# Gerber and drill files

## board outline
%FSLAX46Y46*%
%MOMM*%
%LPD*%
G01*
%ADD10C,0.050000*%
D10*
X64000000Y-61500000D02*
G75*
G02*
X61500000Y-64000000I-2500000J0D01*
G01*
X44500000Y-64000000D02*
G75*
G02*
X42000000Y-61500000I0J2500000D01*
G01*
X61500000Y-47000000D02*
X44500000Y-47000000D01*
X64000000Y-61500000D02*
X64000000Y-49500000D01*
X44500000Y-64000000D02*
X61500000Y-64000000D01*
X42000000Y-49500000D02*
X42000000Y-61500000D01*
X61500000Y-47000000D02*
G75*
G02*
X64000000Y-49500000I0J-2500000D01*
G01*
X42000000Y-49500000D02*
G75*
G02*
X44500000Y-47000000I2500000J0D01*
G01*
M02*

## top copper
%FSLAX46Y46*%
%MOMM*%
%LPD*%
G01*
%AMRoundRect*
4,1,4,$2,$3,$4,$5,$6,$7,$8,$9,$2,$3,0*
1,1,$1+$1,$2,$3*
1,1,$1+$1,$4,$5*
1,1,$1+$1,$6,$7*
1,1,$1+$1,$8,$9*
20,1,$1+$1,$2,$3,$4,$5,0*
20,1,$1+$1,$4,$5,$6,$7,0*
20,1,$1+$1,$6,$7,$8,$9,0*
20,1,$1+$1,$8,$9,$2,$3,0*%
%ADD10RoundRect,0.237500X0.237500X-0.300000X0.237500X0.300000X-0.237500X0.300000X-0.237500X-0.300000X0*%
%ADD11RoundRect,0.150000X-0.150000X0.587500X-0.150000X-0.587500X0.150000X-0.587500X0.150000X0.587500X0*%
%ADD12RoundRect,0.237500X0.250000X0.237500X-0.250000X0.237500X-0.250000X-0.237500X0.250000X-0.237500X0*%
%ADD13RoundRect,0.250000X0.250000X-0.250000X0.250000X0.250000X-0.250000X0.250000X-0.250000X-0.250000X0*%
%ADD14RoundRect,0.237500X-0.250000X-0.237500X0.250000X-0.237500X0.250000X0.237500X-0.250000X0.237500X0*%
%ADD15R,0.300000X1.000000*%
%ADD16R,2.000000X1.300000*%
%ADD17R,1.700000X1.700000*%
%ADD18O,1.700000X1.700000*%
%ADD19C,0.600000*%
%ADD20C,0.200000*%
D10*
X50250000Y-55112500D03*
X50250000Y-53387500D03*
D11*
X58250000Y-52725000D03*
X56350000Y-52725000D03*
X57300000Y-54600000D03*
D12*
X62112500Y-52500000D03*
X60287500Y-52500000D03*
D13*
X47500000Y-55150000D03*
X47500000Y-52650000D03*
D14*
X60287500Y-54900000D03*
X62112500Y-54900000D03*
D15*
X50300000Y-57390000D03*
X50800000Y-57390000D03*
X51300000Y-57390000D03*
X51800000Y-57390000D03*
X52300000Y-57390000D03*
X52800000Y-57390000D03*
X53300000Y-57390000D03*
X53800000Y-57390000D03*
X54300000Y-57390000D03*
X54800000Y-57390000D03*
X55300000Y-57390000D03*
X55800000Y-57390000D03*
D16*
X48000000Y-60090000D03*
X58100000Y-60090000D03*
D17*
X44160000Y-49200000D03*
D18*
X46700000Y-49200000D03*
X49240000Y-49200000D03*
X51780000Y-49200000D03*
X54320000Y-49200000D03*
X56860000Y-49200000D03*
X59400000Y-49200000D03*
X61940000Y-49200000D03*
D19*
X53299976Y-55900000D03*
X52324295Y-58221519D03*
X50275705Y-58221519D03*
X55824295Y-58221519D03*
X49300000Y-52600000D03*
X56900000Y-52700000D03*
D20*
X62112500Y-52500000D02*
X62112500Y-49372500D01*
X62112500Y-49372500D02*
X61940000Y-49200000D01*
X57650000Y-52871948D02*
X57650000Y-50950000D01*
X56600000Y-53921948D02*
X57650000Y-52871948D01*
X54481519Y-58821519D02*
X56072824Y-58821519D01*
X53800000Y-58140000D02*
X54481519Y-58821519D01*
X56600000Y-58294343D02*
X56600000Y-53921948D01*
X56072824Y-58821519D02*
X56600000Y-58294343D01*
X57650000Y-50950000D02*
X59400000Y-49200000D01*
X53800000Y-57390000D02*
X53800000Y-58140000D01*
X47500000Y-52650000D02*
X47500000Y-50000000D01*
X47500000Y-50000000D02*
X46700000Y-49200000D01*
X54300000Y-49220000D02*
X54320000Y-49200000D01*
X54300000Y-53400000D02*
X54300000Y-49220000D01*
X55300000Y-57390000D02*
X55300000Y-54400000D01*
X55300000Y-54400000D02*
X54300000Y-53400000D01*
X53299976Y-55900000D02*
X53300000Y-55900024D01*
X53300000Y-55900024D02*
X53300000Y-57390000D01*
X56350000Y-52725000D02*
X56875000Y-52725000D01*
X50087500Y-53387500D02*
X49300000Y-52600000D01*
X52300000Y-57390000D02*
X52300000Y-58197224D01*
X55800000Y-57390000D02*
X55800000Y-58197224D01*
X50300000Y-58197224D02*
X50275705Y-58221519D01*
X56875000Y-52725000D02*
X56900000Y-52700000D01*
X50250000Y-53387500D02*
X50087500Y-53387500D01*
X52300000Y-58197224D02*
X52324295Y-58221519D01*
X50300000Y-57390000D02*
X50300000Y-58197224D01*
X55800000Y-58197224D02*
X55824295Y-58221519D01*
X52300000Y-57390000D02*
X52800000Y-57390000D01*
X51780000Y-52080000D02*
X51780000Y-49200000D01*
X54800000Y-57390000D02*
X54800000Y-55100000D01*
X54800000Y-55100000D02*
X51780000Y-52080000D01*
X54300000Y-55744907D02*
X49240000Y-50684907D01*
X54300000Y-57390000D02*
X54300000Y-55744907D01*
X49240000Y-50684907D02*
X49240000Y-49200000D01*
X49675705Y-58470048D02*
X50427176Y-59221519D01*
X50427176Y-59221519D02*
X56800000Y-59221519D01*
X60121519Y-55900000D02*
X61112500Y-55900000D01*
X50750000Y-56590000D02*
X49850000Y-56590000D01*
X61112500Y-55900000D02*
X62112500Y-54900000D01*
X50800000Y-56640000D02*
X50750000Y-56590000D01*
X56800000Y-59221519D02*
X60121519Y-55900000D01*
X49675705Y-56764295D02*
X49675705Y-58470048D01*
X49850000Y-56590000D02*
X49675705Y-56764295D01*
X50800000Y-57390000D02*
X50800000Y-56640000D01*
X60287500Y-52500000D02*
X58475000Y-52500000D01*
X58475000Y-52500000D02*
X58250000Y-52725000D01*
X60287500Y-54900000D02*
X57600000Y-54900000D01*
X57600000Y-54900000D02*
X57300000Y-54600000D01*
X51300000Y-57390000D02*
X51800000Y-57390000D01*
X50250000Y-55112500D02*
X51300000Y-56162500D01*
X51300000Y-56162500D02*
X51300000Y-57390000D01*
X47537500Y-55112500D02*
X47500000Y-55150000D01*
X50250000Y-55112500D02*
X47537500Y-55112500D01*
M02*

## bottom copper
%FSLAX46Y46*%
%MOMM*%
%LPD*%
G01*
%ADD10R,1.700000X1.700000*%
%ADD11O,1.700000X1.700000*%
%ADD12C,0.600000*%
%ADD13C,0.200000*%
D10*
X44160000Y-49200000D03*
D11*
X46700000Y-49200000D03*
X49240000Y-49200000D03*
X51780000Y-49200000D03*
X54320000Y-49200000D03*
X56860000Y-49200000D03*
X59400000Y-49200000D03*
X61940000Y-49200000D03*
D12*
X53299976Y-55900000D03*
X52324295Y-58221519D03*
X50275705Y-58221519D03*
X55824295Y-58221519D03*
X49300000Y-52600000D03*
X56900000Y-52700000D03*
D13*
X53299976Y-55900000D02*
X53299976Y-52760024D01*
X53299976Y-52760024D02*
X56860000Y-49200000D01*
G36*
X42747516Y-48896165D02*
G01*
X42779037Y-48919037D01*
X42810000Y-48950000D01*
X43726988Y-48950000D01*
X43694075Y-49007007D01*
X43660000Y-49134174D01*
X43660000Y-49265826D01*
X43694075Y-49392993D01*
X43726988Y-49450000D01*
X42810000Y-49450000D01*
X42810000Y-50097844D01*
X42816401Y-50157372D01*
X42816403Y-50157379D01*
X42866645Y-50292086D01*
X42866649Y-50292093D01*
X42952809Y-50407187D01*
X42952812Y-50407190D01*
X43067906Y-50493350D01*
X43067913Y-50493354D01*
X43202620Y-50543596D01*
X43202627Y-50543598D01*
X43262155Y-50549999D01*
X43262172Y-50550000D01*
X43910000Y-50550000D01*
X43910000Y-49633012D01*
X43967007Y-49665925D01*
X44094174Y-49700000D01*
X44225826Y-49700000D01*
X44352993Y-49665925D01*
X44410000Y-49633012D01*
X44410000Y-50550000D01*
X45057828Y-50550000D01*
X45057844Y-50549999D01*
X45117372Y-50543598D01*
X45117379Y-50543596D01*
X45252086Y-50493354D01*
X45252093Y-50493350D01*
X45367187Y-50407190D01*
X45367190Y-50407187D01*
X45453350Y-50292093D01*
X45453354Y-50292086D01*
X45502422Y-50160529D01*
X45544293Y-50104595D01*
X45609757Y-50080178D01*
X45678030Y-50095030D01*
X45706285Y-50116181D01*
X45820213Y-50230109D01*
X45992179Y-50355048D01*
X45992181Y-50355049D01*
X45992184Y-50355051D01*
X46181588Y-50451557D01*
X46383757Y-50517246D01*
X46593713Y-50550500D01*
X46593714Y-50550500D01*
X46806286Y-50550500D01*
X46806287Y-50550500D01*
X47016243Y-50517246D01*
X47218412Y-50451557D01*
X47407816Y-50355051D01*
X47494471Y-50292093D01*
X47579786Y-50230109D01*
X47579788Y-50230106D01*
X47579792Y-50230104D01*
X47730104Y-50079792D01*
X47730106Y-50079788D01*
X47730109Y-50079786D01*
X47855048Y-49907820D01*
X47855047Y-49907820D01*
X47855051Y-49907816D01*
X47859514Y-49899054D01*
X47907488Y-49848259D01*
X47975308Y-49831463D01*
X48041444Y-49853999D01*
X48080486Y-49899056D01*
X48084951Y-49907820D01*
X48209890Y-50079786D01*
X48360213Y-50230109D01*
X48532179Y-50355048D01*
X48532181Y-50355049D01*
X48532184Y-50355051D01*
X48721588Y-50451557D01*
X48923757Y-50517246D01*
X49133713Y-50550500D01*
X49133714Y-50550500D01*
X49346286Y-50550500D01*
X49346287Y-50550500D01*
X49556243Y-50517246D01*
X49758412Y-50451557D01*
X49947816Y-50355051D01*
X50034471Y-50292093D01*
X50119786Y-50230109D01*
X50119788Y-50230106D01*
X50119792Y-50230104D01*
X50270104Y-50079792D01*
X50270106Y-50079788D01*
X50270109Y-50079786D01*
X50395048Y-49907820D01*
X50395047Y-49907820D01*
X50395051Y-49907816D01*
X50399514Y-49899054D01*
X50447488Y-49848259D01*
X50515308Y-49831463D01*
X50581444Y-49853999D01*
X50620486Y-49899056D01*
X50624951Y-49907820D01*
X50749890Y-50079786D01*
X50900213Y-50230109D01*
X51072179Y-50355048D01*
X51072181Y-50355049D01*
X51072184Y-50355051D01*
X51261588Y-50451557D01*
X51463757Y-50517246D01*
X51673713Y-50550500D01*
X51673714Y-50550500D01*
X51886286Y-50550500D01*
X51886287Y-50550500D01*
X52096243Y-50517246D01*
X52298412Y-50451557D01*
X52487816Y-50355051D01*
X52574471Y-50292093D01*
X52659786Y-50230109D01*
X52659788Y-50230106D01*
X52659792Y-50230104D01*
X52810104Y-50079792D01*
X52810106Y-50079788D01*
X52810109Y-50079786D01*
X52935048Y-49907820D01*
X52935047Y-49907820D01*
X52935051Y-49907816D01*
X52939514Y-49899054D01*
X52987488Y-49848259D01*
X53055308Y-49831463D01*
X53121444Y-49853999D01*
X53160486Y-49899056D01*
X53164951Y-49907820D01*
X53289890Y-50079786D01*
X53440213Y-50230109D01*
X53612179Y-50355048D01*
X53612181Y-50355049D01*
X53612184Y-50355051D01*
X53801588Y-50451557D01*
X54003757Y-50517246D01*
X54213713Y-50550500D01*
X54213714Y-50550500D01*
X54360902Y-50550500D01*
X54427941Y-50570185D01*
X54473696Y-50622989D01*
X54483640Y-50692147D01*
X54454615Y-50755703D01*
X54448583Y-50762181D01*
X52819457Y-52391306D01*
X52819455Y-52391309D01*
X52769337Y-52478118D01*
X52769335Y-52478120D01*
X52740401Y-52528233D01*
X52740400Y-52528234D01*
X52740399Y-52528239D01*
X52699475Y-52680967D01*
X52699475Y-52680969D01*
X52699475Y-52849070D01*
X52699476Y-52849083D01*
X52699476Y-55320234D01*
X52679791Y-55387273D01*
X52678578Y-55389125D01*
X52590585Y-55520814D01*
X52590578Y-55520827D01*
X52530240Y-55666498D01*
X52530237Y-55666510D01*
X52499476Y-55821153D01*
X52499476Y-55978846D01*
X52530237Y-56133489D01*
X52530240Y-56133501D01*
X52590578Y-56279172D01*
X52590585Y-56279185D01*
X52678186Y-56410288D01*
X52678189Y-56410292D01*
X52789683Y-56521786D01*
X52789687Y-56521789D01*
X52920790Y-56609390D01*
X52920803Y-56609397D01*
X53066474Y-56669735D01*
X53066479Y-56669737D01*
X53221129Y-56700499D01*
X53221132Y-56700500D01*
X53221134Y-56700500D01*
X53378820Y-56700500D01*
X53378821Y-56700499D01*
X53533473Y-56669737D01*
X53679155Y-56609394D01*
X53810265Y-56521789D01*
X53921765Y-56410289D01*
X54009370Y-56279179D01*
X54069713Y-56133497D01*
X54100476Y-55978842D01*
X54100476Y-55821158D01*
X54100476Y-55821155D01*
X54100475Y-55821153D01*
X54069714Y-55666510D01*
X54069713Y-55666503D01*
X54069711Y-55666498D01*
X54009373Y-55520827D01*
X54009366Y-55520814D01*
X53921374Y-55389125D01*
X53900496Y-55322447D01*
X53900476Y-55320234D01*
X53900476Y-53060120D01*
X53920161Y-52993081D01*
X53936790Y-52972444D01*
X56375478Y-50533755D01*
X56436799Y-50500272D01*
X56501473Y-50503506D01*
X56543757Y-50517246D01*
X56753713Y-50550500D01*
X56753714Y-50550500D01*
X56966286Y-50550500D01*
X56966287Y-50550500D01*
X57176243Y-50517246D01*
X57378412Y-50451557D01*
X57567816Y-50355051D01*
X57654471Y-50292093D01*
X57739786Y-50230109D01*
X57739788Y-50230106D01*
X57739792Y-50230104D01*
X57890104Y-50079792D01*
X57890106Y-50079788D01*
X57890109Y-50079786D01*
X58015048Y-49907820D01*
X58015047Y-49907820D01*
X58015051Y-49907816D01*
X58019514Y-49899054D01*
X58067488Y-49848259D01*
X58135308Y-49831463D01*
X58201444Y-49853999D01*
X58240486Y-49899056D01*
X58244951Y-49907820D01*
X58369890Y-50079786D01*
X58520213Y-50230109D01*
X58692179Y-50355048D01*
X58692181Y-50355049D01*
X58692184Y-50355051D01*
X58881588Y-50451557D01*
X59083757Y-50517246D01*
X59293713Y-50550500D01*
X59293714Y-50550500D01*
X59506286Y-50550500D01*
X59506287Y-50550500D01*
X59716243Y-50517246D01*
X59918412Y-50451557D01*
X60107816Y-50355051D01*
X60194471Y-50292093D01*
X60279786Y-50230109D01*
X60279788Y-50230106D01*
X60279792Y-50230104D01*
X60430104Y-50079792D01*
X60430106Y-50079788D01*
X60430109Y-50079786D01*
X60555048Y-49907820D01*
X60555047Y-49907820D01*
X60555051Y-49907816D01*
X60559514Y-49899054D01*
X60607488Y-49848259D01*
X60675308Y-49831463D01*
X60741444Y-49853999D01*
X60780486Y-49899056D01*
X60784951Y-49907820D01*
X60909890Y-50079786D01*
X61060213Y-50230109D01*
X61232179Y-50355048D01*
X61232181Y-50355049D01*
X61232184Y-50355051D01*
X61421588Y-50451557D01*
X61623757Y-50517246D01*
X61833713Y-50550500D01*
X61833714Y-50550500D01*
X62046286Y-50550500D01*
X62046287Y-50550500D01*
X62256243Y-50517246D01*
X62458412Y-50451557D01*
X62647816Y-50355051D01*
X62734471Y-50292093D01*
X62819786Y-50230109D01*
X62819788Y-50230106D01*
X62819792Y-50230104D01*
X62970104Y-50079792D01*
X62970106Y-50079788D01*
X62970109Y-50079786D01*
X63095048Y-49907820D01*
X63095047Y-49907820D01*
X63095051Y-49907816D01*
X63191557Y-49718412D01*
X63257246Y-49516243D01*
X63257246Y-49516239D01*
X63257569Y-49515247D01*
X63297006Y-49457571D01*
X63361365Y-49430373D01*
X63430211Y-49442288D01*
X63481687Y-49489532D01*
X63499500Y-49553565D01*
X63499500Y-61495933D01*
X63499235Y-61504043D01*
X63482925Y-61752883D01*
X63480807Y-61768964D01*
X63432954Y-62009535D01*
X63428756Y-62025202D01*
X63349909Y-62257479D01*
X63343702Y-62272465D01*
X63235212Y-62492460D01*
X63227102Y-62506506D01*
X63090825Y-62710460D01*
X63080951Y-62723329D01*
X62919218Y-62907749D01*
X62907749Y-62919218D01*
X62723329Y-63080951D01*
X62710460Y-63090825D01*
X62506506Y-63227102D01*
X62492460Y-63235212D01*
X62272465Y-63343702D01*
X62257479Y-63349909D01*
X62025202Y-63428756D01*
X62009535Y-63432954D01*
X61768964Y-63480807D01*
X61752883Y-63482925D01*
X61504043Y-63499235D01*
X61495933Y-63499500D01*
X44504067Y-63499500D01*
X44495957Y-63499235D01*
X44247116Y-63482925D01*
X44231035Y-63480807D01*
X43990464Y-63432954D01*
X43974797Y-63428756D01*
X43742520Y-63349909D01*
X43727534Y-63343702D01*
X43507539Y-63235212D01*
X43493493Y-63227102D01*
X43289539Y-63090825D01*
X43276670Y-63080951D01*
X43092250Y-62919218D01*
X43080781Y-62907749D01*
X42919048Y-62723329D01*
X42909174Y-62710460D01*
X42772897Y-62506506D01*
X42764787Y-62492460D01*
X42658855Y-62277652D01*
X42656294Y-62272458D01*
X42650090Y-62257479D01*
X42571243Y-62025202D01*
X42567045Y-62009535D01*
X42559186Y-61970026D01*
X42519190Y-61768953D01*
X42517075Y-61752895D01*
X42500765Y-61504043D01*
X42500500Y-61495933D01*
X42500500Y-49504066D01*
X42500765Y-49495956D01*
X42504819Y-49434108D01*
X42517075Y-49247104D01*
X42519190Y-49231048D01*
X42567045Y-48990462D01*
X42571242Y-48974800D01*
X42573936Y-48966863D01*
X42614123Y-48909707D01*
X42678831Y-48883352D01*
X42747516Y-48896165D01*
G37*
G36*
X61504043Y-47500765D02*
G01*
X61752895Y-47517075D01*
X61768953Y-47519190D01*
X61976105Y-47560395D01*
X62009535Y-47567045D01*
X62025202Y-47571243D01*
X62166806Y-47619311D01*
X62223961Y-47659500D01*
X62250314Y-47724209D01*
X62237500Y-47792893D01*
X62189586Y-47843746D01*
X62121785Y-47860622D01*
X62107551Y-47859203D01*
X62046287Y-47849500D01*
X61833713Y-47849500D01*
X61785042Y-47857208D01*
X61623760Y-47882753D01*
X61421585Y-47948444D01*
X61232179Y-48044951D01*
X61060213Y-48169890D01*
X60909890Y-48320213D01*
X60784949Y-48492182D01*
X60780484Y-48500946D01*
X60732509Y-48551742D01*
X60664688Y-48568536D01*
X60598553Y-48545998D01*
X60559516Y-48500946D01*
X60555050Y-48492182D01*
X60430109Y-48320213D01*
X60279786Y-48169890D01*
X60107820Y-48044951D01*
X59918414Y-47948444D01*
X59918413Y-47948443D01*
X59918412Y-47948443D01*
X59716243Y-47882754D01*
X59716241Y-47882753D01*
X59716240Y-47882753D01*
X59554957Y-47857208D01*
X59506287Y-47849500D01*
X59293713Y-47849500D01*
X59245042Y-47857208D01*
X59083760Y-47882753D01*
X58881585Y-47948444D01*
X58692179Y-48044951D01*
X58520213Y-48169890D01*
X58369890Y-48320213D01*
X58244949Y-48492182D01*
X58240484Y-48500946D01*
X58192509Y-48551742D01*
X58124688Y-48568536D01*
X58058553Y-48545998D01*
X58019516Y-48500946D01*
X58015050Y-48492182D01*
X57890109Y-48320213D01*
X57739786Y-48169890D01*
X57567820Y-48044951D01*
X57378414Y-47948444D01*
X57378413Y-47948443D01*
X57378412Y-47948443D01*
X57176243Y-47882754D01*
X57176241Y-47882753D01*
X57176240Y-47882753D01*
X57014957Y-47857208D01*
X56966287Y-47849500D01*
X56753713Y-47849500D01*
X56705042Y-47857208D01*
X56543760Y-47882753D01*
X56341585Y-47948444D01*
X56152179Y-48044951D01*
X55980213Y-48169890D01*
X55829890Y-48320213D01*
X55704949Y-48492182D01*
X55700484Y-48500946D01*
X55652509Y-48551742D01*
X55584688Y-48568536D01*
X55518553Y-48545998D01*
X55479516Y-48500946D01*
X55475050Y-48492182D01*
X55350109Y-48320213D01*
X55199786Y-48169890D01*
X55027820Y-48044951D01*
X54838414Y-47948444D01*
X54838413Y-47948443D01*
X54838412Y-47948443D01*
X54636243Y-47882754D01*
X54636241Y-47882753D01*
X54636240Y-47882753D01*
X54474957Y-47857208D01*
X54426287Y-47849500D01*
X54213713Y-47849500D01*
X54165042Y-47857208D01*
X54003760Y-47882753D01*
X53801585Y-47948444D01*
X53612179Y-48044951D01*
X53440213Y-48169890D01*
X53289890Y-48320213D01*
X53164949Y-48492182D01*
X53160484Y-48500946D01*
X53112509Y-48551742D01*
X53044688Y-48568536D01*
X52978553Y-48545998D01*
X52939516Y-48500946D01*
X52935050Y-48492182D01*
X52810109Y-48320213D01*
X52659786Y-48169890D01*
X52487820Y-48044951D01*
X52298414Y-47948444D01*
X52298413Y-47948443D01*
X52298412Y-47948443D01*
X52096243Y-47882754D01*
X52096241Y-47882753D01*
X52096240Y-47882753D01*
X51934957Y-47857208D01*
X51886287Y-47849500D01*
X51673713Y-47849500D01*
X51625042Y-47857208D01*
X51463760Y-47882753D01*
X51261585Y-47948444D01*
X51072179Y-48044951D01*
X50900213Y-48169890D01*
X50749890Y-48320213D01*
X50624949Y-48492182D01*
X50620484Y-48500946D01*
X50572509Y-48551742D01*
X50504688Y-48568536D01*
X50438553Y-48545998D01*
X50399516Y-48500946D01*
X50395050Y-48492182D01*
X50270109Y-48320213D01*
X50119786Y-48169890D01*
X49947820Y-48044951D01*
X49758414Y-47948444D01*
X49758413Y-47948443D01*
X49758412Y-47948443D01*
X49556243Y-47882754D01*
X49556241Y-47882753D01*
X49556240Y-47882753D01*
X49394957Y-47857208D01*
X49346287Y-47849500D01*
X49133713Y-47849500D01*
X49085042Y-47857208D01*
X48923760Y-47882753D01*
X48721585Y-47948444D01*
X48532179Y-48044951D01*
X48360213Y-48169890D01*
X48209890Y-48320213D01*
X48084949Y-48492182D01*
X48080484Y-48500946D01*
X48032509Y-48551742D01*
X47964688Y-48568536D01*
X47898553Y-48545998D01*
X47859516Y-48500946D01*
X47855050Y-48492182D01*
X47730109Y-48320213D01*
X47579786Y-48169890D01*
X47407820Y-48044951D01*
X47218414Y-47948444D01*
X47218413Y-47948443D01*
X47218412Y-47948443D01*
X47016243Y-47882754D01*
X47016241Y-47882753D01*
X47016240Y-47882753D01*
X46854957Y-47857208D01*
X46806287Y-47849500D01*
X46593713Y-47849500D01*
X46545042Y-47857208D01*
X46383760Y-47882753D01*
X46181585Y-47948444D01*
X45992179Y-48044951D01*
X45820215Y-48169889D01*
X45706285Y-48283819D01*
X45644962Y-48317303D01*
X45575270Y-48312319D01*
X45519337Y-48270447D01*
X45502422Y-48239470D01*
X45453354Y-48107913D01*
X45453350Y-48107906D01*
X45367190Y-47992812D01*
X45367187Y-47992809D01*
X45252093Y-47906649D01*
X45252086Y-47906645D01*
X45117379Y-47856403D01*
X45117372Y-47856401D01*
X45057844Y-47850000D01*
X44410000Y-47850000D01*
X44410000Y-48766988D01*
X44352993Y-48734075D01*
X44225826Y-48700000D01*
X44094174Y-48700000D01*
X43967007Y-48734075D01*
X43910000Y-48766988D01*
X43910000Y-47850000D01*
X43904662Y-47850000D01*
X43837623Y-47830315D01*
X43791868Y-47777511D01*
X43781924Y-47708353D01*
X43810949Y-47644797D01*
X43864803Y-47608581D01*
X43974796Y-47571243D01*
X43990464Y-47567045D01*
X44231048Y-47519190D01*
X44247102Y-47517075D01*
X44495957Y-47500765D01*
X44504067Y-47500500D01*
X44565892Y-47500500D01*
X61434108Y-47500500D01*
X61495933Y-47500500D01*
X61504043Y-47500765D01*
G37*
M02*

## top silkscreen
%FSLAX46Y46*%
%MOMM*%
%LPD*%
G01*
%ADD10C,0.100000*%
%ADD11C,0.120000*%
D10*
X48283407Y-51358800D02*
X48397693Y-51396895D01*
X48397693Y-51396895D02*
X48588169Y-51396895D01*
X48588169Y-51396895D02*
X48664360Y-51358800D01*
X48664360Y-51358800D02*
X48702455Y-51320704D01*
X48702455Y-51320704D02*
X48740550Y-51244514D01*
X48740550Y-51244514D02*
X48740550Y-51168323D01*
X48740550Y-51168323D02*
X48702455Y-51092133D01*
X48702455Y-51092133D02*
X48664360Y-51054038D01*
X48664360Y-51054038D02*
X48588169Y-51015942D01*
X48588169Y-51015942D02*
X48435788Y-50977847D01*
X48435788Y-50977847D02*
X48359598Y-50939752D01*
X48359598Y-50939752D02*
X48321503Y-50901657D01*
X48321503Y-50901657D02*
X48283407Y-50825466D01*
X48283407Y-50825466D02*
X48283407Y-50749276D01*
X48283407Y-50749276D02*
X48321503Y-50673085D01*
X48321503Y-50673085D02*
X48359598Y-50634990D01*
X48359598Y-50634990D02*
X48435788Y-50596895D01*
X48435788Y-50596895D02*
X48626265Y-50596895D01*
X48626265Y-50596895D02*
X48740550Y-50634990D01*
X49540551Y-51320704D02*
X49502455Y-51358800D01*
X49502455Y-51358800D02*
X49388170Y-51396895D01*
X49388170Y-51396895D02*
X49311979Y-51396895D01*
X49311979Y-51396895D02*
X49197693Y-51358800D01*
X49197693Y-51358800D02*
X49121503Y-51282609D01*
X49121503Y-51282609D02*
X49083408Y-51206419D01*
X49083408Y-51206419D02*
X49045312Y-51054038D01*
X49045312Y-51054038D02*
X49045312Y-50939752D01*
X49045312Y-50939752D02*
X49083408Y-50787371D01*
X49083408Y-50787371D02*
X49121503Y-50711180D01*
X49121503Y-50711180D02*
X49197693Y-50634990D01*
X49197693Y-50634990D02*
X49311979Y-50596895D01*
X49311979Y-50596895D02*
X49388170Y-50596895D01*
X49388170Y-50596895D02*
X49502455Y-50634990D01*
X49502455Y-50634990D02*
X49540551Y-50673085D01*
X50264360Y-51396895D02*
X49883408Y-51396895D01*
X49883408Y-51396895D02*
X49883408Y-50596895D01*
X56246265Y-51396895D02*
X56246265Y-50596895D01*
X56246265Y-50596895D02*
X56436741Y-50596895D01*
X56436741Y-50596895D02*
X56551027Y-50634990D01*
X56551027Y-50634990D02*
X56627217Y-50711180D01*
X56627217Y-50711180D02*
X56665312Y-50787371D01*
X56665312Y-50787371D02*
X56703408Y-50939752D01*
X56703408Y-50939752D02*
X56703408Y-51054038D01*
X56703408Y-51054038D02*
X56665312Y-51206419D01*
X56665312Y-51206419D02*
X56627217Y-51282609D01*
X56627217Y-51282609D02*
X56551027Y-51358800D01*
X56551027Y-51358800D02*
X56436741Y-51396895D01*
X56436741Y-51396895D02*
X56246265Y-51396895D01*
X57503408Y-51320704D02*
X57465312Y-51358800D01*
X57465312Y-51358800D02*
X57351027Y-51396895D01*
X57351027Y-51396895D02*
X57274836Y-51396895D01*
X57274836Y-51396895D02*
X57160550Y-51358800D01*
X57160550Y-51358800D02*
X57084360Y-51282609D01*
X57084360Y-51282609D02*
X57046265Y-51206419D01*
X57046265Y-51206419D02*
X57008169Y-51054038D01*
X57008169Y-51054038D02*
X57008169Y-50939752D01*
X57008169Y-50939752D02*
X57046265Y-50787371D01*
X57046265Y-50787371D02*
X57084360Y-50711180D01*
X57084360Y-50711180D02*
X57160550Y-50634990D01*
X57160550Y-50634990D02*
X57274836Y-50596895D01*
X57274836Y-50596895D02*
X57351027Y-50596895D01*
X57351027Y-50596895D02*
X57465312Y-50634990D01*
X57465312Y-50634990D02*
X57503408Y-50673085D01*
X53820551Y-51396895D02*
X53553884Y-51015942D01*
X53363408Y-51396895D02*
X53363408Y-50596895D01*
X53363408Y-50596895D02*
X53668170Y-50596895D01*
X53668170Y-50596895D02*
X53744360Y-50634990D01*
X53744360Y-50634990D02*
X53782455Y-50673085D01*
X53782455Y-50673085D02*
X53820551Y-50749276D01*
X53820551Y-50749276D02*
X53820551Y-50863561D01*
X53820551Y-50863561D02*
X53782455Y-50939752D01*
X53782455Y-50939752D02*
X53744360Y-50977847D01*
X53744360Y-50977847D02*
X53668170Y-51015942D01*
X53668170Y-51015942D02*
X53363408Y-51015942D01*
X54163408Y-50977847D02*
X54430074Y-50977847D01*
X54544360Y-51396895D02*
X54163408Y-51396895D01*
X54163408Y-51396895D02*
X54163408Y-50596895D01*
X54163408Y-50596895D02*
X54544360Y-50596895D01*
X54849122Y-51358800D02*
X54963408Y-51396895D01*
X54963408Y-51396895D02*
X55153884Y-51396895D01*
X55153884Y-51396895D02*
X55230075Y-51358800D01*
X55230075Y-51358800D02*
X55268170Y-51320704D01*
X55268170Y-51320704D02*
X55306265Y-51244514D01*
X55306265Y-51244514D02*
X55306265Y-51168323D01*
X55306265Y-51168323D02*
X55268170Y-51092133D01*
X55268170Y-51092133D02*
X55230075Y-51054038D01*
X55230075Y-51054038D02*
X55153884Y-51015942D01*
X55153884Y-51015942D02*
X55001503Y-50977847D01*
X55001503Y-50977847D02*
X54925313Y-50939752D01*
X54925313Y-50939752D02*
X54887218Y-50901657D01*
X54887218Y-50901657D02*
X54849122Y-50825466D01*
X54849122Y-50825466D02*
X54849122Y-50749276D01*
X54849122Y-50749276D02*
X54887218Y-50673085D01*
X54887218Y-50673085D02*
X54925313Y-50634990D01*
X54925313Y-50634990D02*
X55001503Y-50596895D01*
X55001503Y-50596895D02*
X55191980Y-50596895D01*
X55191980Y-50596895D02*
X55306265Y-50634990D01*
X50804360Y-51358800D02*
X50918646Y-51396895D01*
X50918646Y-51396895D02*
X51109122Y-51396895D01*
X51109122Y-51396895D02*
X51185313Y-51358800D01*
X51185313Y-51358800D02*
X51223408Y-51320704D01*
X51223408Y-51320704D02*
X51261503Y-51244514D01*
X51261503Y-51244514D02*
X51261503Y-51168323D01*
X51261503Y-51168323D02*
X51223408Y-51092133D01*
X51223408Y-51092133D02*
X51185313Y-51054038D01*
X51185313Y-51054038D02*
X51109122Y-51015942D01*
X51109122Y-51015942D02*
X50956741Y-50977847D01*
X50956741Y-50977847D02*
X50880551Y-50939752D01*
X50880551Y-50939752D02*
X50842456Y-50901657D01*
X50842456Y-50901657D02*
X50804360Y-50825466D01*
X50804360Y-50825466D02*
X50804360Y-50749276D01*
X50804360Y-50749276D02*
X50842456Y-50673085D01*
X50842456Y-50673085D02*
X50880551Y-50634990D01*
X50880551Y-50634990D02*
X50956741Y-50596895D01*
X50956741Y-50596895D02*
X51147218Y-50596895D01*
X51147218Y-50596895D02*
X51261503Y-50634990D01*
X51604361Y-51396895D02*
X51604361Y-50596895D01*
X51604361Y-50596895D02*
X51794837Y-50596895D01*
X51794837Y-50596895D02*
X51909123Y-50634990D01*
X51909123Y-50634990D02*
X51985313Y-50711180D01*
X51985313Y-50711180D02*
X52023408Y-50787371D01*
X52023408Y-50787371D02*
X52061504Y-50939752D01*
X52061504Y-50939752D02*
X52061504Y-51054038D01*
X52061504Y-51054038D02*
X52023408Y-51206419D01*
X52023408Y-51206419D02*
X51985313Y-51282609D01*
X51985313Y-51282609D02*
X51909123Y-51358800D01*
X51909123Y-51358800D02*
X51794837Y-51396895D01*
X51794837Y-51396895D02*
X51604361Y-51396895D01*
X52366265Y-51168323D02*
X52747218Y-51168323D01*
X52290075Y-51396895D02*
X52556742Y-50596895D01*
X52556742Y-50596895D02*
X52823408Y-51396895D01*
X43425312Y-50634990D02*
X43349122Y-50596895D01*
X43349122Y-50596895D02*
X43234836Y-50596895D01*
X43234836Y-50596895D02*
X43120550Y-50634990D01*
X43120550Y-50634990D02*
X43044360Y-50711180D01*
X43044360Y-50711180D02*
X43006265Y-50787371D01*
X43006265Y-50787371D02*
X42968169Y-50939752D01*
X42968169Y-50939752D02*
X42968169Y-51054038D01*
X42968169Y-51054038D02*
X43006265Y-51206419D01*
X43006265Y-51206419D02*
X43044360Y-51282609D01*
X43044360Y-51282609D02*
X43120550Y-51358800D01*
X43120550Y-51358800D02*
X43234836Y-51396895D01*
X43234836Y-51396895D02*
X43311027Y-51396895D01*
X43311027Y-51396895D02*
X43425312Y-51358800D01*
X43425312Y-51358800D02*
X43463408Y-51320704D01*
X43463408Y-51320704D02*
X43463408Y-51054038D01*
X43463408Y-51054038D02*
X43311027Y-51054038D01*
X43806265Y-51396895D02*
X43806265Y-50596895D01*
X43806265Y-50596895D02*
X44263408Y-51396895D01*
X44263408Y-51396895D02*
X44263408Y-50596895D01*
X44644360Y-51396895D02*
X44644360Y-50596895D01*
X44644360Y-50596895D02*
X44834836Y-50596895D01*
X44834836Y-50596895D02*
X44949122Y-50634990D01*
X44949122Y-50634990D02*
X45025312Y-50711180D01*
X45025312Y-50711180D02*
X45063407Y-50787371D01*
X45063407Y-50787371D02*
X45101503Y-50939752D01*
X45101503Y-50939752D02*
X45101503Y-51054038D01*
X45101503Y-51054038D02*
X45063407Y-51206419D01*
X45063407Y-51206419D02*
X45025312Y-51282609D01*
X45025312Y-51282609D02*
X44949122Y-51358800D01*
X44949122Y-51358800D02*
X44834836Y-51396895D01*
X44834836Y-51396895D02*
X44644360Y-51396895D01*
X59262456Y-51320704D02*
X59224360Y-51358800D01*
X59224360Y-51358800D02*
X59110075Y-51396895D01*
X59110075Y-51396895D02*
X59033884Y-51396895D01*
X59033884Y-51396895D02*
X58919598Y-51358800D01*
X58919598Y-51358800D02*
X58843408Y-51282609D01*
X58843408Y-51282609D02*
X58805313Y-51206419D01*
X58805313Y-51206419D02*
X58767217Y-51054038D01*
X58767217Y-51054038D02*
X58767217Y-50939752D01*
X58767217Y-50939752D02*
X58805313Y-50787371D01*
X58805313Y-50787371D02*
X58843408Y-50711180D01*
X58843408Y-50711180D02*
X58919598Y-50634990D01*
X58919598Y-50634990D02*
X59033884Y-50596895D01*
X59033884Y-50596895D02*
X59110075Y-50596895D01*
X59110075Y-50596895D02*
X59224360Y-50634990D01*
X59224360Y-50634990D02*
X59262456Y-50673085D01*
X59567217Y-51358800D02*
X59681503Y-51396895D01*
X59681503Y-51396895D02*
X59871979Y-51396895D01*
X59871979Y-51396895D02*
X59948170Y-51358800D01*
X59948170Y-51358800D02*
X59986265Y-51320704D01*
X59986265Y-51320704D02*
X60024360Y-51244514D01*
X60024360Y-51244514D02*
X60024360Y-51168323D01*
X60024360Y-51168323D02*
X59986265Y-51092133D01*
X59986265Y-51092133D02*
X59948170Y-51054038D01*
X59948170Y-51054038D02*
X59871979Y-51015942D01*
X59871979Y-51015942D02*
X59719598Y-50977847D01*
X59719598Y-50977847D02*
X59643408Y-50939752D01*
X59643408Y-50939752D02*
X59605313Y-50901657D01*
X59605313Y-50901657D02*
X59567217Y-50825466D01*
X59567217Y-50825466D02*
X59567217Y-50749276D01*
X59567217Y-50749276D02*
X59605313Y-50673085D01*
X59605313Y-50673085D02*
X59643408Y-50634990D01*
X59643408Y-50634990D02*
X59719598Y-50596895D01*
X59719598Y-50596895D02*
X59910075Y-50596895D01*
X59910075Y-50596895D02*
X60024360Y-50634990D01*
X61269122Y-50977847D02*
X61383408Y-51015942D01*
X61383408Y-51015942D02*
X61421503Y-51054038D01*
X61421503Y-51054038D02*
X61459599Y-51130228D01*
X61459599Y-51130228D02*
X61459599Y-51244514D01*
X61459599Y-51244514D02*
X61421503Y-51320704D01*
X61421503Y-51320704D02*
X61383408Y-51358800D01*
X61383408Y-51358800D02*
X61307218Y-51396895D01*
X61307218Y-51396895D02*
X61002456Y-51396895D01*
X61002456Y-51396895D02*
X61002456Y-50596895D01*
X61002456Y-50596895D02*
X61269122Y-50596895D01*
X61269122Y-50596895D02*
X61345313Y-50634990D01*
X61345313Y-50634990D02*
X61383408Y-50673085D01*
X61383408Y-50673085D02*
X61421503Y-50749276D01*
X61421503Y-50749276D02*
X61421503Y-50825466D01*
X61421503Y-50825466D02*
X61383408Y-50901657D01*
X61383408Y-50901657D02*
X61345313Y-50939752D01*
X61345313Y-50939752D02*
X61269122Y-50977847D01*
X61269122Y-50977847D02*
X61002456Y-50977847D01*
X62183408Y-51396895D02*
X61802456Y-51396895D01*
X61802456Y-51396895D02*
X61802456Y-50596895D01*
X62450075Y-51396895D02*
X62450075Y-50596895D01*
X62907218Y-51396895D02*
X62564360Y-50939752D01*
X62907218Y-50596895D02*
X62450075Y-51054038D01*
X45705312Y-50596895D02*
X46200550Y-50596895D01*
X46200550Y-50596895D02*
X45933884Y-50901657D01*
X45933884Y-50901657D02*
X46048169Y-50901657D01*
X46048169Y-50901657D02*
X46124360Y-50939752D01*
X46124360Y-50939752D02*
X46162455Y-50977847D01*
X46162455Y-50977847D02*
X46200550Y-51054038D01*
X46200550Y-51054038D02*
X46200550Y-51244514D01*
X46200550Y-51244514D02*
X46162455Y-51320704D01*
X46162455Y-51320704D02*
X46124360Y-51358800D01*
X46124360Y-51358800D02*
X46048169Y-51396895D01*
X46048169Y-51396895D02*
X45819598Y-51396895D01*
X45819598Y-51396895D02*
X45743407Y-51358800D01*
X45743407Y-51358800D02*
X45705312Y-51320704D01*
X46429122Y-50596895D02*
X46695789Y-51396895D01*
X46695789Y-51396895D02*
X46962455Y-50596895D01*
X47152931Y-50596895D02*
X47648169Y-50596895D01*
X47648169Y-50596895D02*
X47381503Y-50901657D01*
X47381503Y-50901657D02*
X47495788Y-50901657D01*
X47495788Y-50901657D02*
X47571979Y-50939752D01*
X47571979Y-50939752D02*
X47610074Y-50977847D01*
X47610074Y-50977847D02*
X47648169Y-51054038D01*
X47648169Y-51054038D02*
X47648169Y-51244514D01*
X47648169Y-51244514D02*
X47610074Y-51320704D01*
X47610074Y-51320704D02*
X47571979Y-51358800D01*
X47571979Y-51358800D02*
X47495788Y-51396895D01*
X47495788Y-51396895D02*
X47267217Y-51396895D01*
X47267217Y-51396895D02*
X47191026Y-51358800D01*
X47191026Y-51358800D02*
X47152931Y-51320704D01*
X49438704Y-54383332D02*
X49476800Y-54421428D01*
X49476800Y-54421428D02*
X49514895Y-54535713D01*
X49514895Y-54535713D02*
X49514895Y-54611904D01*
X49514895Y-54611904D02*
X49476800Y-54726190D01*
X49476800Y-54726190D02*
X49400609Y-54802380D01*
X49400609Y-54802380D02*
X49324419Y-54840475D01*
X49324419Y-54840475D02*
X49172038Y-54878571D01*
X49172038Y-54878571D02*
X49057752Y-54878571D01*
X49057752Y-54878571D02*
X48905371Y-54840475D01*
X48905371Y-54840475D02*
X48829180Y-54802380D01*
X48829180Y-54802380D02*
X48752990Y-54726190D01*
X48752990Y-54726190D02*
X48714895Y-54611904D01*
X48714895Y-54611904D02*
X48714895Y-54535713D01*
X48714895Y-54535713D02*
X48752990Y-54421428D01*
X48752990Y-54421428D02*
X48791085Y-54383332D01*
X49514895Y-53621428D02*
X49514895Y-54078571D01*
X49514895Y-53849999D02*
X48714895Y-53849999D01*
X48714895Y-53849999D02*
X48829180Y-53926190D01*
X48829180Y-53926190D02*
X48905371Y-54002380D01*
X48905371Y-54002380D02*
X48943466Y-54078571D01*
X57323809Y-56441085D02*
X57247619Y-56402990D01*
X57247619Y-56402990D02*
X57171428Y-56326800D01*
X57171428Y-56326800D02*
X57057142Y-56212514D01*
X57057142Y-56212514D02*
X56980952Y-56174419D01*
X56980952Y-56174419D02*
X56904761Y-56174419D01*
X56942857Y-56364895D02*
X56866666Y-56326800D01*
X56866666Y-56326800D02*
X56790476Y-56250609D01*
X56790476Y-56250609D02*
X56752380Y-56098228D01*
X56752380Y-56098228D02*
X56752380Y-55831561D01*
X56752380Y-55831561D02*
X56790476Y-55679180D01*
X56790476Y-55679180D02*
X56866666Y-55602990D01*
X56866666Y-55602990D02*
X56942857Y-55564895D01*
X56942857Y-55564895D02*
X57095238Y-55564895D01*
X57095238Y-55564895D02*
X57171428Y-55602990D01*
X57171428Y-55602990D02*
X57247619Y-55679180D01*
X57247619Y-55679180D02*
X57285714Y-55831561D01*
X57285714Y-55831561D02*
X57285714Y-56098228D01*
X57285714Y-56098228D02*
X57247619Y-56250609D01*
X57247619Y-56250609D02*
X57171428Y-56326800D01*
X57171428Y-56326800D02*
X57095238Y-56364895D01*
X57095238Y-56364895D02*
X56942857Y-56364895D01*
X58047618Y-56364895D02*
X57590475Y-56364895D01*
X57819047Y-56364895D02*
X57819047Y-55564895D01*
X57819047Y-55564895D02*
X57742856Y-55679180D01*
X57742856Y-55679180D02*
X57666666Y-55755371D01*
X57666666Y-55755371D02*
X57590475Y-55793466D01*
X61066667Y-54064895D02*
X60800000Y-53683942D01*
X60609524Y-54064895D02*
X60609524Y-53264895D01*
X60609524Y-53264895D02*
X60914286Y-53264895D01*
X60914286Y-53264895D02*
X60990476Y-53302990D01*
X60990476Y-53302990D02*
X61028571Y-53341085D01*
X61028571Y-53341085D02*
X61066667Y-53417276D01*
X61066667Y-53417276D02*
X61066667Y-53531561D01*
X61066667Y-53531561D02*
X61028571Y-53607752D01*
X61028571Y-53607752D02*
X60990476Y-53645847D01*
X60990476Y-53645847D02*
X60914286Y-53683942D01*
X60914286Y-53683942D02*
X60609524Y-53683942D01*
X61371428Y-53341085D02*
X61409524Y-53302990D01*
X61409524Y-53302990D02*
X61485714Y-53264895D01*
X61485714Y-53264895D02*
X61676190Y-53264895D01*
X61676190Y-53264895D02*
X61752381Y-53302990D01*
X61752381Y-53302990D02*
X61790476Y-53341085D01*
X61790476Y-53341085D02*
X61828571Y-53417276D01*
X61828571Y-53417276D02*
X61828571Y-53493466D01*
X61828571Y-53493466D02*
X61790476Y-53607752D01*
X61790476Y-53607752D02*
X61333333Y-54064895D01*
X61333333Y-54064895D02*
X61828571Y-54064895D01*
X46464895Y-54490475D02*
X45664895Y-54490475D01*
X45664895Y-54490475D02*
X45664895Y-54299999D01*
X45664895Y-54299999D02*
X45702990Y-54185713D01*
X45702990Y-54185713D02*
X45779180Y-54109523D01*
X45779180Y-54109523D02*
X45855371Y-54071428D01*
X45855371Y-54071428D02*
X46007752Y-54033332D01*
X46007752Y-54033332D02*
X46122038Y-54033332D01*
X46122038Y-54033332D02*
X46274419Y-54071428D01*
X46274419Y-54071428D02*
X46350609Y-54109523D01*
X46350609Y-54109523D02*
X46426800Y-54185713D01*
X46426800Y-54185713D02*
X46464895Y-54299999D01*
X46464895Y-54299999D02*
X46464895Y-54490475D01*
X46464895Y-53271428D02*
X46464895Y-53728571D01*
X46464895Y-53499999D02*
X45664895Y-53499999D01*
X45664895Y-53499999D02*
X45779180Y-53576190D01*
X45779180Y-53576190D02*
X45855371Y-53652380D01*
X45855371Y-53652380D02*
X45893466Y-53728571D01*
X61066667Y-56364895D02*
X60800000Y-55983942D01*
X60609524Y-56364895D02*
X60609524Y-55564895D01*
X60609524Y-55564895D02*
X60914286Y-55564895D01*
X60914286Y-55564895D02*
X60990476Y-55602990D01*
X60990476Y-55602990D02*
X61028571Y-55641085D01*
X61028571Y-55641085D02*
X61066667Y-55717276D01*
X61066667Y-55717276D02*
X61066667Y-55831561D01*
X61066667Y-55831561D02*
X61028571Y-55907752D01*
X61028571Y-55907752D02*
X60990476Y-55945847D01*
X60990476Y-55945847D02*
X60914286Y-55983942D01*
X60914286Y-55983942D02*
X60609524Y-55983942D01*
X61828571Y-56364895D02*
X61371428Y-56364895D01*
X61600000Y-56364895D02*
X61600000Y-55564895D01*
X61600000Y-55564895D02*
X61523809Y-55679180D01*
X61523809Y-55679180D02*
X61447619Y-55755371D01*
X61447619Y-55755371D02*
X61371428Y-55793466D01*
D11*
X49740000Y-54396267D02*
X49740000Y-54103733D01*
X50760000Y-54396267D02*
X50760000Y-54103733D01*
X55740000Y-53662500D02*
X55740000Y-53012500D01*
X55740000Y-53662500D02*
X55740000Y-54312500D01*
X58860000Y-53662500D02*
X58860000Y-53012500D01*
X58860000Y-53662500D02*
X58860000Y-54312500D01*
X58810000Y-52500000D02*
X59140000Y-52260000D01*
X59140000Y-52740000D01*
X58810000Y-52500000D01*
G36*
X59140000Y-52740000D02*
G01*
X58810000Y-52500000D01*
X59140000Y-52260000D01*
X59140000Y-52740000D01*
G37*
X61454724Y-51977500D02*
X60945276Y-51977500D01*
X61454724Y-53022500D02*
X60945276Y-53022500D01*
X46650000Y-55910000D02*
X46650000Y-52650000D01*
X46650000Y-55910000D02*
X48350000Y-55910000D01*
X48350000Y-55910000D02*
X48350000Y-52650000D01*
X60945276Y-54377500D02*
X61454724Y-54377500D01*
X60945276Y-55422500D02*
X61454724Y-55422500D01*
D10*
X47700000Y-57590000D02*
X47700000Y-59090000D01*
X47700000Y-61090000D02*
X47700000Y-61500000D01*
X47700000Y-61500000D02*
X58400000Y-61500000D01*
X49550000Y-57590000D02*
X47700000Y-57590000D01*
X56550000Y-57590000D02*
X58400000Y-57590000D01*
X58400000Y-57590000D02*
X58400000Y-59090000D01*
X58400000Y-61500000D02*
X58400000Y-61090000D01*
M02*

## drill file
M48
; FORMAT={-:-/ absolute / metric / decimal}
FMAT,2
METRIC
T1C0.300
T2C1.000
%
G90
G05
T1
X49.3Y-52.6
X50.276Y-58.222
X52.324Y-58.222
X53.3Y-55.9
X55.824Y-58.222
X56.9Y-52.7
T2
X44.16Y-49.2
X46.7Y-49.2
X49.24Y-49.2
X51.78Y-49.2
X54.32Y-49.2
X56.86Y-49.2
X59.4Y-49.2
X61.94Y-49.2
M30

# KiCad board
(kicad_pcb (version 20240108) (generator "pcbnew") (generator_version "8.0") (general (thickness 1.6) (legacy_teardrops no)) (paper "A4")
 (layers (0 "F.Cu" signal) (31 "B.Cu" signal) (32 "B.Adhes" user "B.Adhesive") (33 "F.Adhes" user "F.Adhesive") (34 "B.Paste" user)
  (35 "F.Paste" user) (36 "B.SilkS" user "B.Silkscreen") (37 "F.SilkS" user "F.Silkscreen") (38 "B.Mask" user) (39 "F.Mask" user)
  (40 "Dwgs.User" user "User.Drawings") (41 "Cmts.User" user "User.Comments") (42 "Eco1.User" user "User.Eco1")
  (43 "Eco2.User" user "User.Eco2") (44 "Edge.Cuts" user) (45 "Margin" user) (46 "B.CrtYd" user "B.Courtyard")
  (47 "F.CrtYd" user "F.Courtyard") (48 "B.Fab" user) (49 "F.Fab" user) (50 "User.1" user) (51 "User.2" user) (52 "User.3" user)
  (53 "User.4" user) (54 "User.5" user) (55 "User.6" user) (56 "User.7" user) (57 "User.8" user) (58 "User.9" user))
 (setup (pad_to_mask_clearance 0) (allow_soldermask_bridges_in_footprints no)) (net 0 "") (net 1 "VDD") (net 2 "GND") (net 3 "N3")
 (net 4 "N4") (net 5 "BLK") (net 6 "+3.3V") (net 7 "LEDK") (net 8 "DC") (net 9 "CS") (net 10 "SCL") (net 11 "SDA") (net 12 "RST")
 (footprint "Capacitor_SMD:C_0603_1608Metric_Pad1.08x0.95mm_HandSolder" (layer "F.Cu") (at 50.25 54.25 90)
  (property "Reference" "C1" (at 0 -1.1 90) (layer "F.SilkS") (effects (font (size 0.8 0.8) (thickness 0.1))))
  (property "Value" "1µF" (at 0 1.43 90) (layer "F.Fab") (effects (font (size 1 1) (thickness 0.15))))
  (fp_line (start -0.146267 -0.51) (end 0.146267 -0.51) (stroke (width 0.12) (type solid)) (layer "F.SilkS"))
  (fp_line (start -0.146267 0.51) (end 0.146267 0.51) (stroke (width 0.12) (type solid)) (layer "F.SilkS"))
  (pad "1" smd roundrect (at -0.8625 0 90) (size 1.075 0.95) (layers "F.Cu" "F.Paste" "F.Mask") (roundrect_rratio 0.25) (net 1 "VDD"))
  (pad "2" smd roundrect (at 0.8625 0 90) (size 1.075 0.95) (layers "F.Cu" "F.Paste" "F.Mask") (roundrect_rratio 0.25) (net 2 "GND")))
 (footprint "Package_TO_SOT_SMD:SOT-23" (layer "F.Cu") (at 57.3 53.6625 -90)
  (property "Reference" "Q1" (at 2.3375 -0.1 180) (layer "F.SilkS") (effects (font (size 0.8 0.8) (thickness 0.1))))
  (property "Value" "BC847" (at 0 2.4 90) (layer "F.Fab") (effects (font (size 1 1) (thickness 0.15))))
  (fp_line (start 0 1.56) (end -0.65 1.56) (stroke (width 0.12) (type solid)) (layer "F.SilkS"))
  (fp_line (start 0 1.56) (end 0.65 1.56) (stroke (width 0.12) (type solid)) (layer "F.SilkS"))
  (fp_line (start 0 -1.56) (end -0.65 -1.56) (stroke (width 0.12) (type solid)) (layer "F.SilkS"))
  (fp_line (start 0 -1.56) (end 0.65 -1.56) (stroke (width 0.12) (type solid)) (layer "F.SilkS"))
  (fp_poly
   (pts (xy -1.1625 -1.51) (xy -1.4025 -1.84) (xy -0.9225 -1.84) (xy -1.1625 -1.51)) (stroke (width 0.12) (type solid)) (fill solid)
   (layer "F.SilkS"))
  (pad "1" smd roundrect (at -0.9375 -0.95 270) (size 1.475 0.6) (layers "F.Cu" "F.Paste" "F.Mask") (roundrect_rratio 0.25) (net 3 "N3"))
  (pad "2" smd roundrect (at -0.9375 0.95 270) (size 1.475 0.6) (layers "F.Cu" "F.Paste" "F.Mask") (roundrect_rratio 0.25) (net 2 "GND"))
  (pad "3" smd roundrect (at 0.9375 0 270) (size 1.475 0.6) (layers "F.Cu" "F.Paste" "F.Mask") (roundrect_rratio 0.25) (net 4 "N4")))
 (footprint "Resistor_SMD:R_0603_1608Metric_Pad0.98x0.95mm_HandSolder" (layer "F.Cu") (at 61.2 52.5 180)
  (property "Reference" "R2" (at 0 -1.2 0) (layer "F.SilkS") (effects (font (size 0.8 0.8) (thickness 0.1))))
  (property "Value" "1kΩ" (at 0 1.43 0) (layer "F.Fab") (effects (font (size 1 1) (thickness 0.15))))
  (fp_line (start -0.254724 0.5225) (end 0.254724 0.5225) (stroke (width 0.12) (type solid)) (layer "F.SilkS"))
  (fp_line (start -0.254724 -0.5225) (end 0.254724 -0.5225) (stroke (width 0.12) (type solid)) (layer "F.SilkS"))
  (pad "1" smd roundrect (at -0.9125 0 180) (size 0.975 0.95) (layers "F.Cu" "F.Paste" "F.Mask") (roundrect_rratio 0.25) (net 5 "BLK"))
  (pad "2" smd roundrect (at 0.9125 0 180) (size 0.975 0.95) (layers "F.Cu" "F.Paste" "F.Mask") (roundrect_rratio 0.25) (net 3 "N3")))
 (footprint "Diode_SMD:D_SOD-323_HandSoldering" (layer "F.Cu") (at 47.5 53.9 90)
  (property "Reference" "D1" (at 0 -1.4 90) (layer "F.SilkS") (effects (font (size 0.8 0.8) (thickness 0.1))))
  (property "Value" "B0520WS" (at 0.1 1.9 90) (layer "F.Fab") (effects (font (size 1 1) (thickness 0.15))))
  (fp_line (start -2.01 -0.85) (end 1.25 -0.85) (stroke (width 0.12) (type solid)) (layer "F.SilkS"))
  (fp_line (start -2.01 -0.85) (end -2.01 0.85) (stroke (width 0.12) (type solid)) (layer "F.SilkS"))
  (fp_line (start -2.01 0.85) (end 1.25 0.85) (stroke (width 0.12) (type solid)) (layer "F.SilkS"))
  (pad "1" smd roundrect (at -1.25 0 90) (size 1 1) (layers "F.Cu" "F.Paste" "F.Mask") (roundrect_rratio 0.25) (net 1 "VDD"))
  (pad "2" smd roundrect (at 1.25 0 90) (size 1 1) (layers "F.Cu" "F.Paste" "F.Mask") (roundrect_rratio 0.25) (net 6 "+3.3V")))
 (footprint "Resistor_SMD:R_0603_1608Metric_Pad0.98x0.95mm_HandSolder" (layer "F.Cu") (at 61.2 54.9)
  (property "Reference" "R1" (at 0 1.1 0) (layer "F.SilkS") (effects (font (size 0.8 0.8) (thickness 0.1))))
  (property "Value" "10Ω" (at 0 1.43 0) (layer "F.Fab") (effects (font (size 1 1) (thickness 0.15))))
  (fp_line (start -0.254724 -0.5225) (end 0.254724 -0.5225) (stroke (width 0.12) (type solid)) (layer "F.SilkS"))
  (fp_line (start -0.254724 0.5225) (end 0.254724 0.5225) (stroke (width 0.12) (type solid)) (layer "F.SilkS"))
  (pad "1" smd roundrect (at -0.9125 0) (size 0.975 0.95) (layers "F.Cu" "F.Paste" "F.Mask") (roundrect_rratio 0.25) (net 4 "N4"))
  (pad "2" smd roundrect (at 0.9125 0) (size 0.975 0.95) (layers "F.Cu" "F.Paste" "F.Mask") (roundrect_rratio 0.25) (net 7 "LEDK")))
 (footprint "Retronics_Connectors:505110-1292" (layer "F.Cu") (at 53.05 59.845)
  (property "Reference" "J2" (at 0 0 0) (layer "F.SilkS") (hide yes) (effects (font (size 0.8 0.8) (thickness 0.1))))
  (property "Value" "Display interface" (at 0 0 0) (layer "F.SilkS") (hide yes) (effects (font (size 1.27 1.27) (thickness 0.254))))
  (fp_line (start -5.35 -2.255) (end -5.35 -0.755) (stroke (width 0.1) (type solid)) (layer "F.SilkS"))
  (fp_line (start -5.35 1.245) (end -5.35 1.655) (stroke (width 0.1) (type solid)) (layer "F.SilkS"))
  (fp_line (start -5.35 1.655) (end 5.35 1.655) (stroke (width 0.1) (type solid)) (layer "F.SilkS"))
  (fp_line (start -3.5 -2.255) (end -5.35 -2.255) (stroke (width 0.1) (type solid)) (layer "F.SilkS"))
  (fp_line (start 3.5 -2.255) (end 5.35 -2.255) (stroke (width 0.1) (type solid)) (layer "F.SilkS"))
  (fp_line (start 5.35 -2.255) (end 5.35 -0.755) (stroke (width 0.1) (type solid)) (layer "F.SilkS"))
  (fp_line (start 5.35 1.655) (end 5.35 1.245) (stroke (width 0.1) (type solid)) (layer "F.SilkS"))
  (pad "1" smd rect (at -2.75 -2.455) (size 0.3 1) (layers "F.Cu" "F.Paste" "F.Mask") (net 2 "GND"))
  (pad "2" smd rect (at -2.25 -2.455) (size 0.3 1) (layers "F.Cu" "F.Paste" "F.Mask") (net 7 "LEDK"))
  (pad "3" smd rect (at -1.75 -2.455) (size 0.3 1) (layers "F.Cu" "F.Paste" "F.Mask") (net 1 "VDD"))
  (pad "4" smd rect (at -1.25 -2.455) (size 0.3 1) (layers "F.Cu" "F.Paste" "F.Mask") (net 1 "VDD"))
  (pad "5" smd rect (at -0.75 -2.455) (size 0.3 1) (layers "F.Cu" "F.Paste" "F.Mask") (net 2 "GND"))
  (pad "6" smd rect (at -0.25 -2.455) (size 0.3 1) (layers "F.Cu" "F.Paste" "F.Mask") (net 2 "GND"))
  (pad "7" smd rect (at 0.25 -2.455) (size 0.3 1) (layers "F.Cu" "F.Paste" "F.Mask") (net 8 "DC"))
  (pad "8" smd rect (at 0.75 -2.455) (size 0.3 1) (layers "F.Cu" "F.Paste" "F.Mask") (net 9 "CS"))
  (pad "9" smd rect (at 1.25 -2.455) (size 0.3 1) (layers "F.Cu" "F.Paste" "F.Mask") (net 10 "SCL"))
  (pad "10" smd rect (at 1.75 -2.455) (size 0.3 1) (layers "F.Cu" "F.Paste" "F.Mask") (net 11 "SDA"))
  (pad "11" smd rect (at 2.25 -2.455) (size 0.3 1) (layers "F.Cu" "F.Paste" "F.Mask") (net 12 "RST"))
  (pad "12" smd rect (at 2.75 -2.455) (size 0.3 1) (layers "F.Cu" "F.Paste" "F.Mask") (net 2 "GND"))
  (pad "MP1" smd rect (at -5.05 0.245 90) (size 1.3 2) (layers "F.Cu" "F.Paste" "F.Mask"))
  (pad "MP2" smd rect (at 5.05 0.245 90) (size 1.3 2) (layers "F.Cu" "F.Paste" "F.Mask")))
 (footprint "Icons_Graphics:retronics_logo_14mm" (layer "B.Cu") (at 52.996672 54.8 180)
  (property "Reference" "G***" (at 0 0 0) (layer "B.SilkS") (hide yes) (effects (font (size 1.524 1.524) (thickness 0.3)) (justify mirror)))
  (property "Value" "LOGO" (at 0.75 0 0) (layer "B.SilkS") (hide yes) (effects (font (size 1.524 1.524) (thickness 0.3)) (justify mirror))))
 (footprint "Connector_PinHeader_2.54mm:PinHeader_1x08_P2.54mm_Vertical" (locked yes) (layer "B.Cu") (at 44.16 49.2 -90)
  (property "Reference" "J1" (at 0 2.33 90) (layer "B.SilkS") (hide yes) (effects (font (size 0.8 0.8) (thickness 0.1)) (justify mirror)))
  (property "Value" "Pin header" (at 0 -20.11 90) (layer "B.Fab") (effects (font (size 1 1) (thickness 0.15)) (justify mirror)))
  (pad "1" thru_hole rect (at 0 0 270) (size 1.7 1.7) (drill 1) (layers "*.Cu" "*.Mask") (remove_unused_layers no) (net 2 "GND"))
  (pad "2" thru_hole oval (at 0 -2.54 270) (size 1.7 1.7) (drill 1) (layers "*.Cu" "*.Mask") (remove_unused_layers no) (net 6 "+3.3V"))
  (pad "3" thru_hole oval (at 0 -5.08 270) (size 1.7 1.7) (drill 1) (layers "*.Cu" "*.Mask") (remove_unused_layers no) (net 10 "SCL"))
  (pad "4" thru_hole oval (at 0 -7.62 270) (size 1.7 1.7) (drill 1) (layers "*.Cu" "*.Mask") (remove_unused_layers no) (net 11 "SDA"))
  (pad "5" thru_hole oval (at 0 -10.16 270) (size 1.7 1.7) (drill 1) (layers "*.Cu" "*.Mask") (remove_unused_layers no) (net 12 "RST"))
  (pad "6" thru_hole oval (at 0 -12.7 270) (size 1.7 1.7) (drill 1) (layers "*.Cu" "*.Mask") (remove_unused_layers no) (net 8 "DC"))
  (pad "7" thru_hole oval (at 0 -15.24 270) (size 1.7 1.7) (drill 1) (layers "*.Cu" "*.Mask") (remove_unused_layers no) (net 9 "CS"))
  (pad "8" thru_hole oval (at 0 -17.78 270) (size 1.7 1.7) (drill 1) (layers "*.Cu" "*.Mask") (remove_unused_layers no) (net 5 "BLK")))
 (gr_arc (start 64 61.5) (mid 63.267767 63.267767) (end 61.5 64) (stroke (width 0.05) (type default)) (layer "Edge.Cuts"))
 (gr_arc (start 44.5 64) (mid 42.732233 63.267767) (end 42 61.5) (stroke (width 0.05) (type default)) (layer "Edge.Cuts"))
 (gr_line (start 61.5 47) (end 44.5 47) (stroke (width 0.05) (type default)) (layer "Edge.Cuts"))
 (gr_line (start 64 61.5) (end 64 49.5) (stroke (width 0.05) (type default)) (layer "Edge.Cuts"))
 (gr_line (start 44.5 64) (end 61.5 64) (stroke (width 0.05) (type default)) (layer "Edge.Cuts"))
 (gr_line (start 42 49.5) (end 42 61.5) (stroke (width 0.05) (type default)) (layer "Edge.Cuts"))
 (gr_arc (start 61.5 47) (mid 63.267767 47.732233) (end 64 49.5) (stroke (width 0.05) (type default)) (layer "Edge.Cuts"))
 (gr_arc (start 42 49.5) (mid 42.732233 47.732233) (end 44.5 47) (stroke (width 0.05) (type default)) (layer "Edge.Cuts"))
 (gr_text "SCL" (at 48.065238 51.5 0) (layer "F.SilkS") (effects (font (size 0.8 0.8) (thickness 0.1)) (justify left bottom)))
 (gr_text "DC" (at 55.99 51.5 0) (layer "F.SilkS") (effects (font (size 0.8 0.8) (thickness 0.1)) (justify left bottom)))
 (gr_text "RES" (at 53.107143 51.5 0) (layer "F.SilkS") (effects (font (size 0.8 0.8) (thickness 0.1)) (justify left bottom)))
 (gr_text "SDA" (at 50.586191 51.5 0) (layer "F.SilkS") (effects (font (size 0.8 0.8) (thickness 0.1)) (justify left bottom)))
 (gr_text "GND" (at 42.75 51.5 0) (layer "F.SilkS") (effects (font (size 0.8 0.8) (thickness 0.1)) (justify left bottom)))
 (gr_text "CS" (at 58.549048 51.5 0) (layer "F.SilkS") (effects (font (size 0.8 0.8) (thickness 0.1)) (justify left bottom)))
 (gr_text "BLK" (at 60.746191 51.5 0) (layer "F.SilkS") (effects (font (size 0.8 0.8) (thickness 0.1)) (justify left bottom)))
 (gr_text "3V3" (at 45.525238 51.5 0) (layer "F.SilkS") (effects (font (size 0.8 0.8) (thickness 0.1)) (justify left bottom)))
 (segment (start 62.1125 52.5) (end 62.1125 49.3725) (width 0.2) (layer "F.Cu") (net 5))
 (segment (start 62.1125 49.3725) (end 61.94 49.2) (width 0.2) (layer "F.Cu") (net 5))
 (segment (start 57.65 52.871948) (end 57.65 50.95) (width 0.2) (layer "F.Cu") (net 9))
 (segment (start 56.6 53.921948) (end 57.65 52.871948) (width 0.2) (layer "F.Cu") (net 9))
 (segment (start 54.481519 58.821519) (end 56.072824 58.821519) (width 0.2) (layer "F.Cu") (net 9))
 (segment (start 53.8 58.14) (end 54.481519 58.821519) (width 0.2) (layer "F.Cu") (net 9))
 (segment (start 56.6 58.294343) (end 56.6 53.921948) (width 0.2) (layer "F.Cu") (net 9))
 (segment (start 56.072824 58.821519) (end 56.6 58.294343) (width 0.2) (layer "F.Cu") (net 9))
 (segment (start 57.65 50.95) (end 59.4 49.2) (width 0.2) (layer "F.Cu") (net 9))
 (segment (start 53.8 57.39) (end 53.8 58.14) (width 0.2) (layer "F.Cu") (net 9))
 (segment (start 47.5 52.65) (end 47.5 50) (width 0.2) (layer "F.Cu") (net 6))
 (segment (start 47.5 50) (end 46.7 49.2) (width 0.2) (layer "F.Cu") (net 6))
 (segment (start 54.3 49.22) (end 54.32 49.2) (width 0.2) (layer "F.Cu") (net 12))
 (segment (start 54.3 53.4) (end 54.3 49.22) (width 0.2) (layer "F.Cu") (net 12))
 (segment (start 55.3 57.39) (end 55.3 54.4) (width 0.2) (layer "F.Cu") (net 12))
 (segment (start 55.3 54.4) (end 54.3 53.4) (width 0.2) (layer "F.Cu") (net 12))
 (segment (start 53.299976 55.9) (end 53.3 55.900024) (width 0.2) (layer "F.Cu") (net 8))
 (segment (start 53.3 55.900024) (end 53.3 57.39) (width 0.2) (layer "F.Cu") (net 8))
 (via (at 53.299976 55.9) (size 0.6) (drill 0.3) (layers "F.Cu" "B.Cu") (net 8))
 (segment (start 53.299976 55.9) (end 53.299976 52.760024) (width 0.2) (layer "B.Cu") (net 8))
 (segment (start 53.299976 52.760024) (end 56.86 49.2) (width 0.2) (layer "B.Cu") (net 8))
 (segment (start 56.35 52.725) (end 56.875 52.725) (width 0.2) (layer "F.Cu") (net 2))
 (segment (start 50.0875 53.3875) (end 49.3 52.6) (width 0.2) (layer "F.Cu") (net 2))
 (segment (start 52.3 57.39) (end 52.3 58.197224) (width 0.2) (layer "F.Cu") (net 2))
 (segment (start 55.8 57.39) (end 55.8 58.197224) (width 0.2) (layer "F.Cu") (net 2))
 (segment (start 50.3 58.197224) (end 50.275705 58.221519) (width 0.2) (layer "F.Cu") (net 2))
 (segment (start 56.875 52.725) (end 56.9 52.7) (width 0.2) (layer "F.Cu") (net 2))
 (segment (start 50.25 53.3875) (end 50.0875 53.3875) (width 0.2) (layer "F.Cu") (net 2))
 (segment (start 52.3 58.197224) (end 52.324295 58.221519) (width 0.2) (layer "F.Cu") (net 2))
 (segment (start 50.3 57.39) (end 50.3 58.197224) (width 0.2) (layer "F.Cu") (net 2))
 (segment (start 55.8 58.197224) (end 55.824295 58.221519) (width 0.2) (layer "F.Cu") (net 2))
 (segment (start 52.3 57.39) (end 52.8 57.39) (width 0.2) (layer "F.Cu") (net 2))
 (via (at 52.324295 58.221519) (size 0.6) (drill 0.3) (layers "F.Cu" "B.Cu") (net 2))
 (via (at 50.275705 58.221519) (size 0.6) (drill 0.3) (layers "F.Cu" "B.Cu") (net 2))
 (via (at 55.824295 58.221519) (size 0.6) (drill 0.3) (layers "F.Cu" "B.Cu") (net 2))
 (via (at 49.3 52.6) (size 0.6) (drill 0.3) (layers "F.Cu" "B.Cu") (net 2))
 (via (at 56.9 52.7) (size 0.6) (drill 0.3) (layers "F.Cu" "B.Cu") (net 2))
 (segment (start 51.78 52.08) (end 51.78 49.2) (width 0.2) (layer "F.Cu") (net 11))
 (segment (start 54.8 57.39) (end 54.8 55.1) (width 0.2) (layer "F.Cu") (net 11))
 (segment (start 54.8 55.1) (end 51.78 52.08) (width 0.2) (layer "F.Cu") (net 11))
 (segment (start 54.3 55.744907) (end 49.24 50.684907) (width 0.2) (layer "F.Cu") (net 10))
 (segment (start 54.3 57.39) (end 54.3 55.744907) (width 0.2) (layer "F.Cu") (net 10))
 (segment (start 49.24 50.684907) (end 49.24 49.2) (width 0.2) (layer "F.Cu") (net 10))
 (segment (start 49.675705 58.470048) (end 50.427176 59.221519) (width 0.2) (layer "F.Cu") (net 7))
 (segment (start 50.427176 59.221519) (end 56.8 59.221519) (width 0.2) (layer "F.Cu") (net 7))
 (segment (start 60.121519 55.9) (end 61.1125 55.9) (width 0.2) (layer "F.Cu") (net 7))
 (segment (start 50.75 56.59) (end 49.85 56.59) (width 0.2) (layer "F.Cu") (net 7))
 (segment (start 61.1125 55.9) (end 62.1125 54.9) (width 0.2) (layer "F.Cu") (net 7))
 (segment (start 50.8 56.64) (end 50.75 56.59) (width 0.2) (layer "F.Cu") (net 7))
 (segment (start 56.8 59.221519) (end 60.121519 55.9) (width 0.2) (layer "F.Cu") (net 7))
 (segment (start 49.675705 56.764295) (end 49.675705 58.470048) (width 0.2) (layer "F.Cu") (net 7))
 (segment (start 49.85 56.59) (end 49.675705 56.764295) (width 0.2) (layer "F.Cu") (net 7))
 (segment (start 50.8 57.39) (end 50.8 56.64) (width 0.2) (layer "F.Cu") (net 7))
 (segment (start 60.2875 52.5) (end 58.475 52.5) (width 0.2) (layer "F.Cu") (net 3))
 (segment (start 58.475 52.5) (end 58.25 52.725) (width 0.2) (layer "F.Cu") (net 3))
 (segment (start 60.2875 54.9) (end 57.6 54.9) (width 0.2) (layer "F.Cu") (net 4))
 (segment (start 57.6 54.9) (end 57.3 54.6) (width 0.2) (layer "F.Cu") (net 4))
 (segment (start 51.3 57.39) (end 51.8 57.39) (width 0.2) (layer "F.Cu") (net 1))
 (segment (start 50.25 55.1125) (end 51.3 56.1625) (width 0.2) (layer "F.Cu") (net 1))
 (segment (start 51.3 56.1625) (end 51.3 57.39) (width 0.2) (layer "F.Cu") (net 1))
 (segment (start 47.5375 55.1125) (end 47.5 55.15) (width 0.2) (layer "F.Cu") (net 1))
 (segment (start 50.25 55.1125) (end 47.5375 55.1125) (width 0.2) (layer "F.Cu") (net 1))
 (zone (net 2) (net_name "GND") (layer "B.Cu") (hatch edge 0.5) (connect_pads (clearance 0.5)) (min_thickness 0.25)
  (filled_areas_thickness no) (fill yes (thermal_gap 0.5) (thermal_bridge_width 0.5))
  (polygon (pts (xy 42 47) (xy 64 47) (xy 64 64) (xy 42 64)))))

